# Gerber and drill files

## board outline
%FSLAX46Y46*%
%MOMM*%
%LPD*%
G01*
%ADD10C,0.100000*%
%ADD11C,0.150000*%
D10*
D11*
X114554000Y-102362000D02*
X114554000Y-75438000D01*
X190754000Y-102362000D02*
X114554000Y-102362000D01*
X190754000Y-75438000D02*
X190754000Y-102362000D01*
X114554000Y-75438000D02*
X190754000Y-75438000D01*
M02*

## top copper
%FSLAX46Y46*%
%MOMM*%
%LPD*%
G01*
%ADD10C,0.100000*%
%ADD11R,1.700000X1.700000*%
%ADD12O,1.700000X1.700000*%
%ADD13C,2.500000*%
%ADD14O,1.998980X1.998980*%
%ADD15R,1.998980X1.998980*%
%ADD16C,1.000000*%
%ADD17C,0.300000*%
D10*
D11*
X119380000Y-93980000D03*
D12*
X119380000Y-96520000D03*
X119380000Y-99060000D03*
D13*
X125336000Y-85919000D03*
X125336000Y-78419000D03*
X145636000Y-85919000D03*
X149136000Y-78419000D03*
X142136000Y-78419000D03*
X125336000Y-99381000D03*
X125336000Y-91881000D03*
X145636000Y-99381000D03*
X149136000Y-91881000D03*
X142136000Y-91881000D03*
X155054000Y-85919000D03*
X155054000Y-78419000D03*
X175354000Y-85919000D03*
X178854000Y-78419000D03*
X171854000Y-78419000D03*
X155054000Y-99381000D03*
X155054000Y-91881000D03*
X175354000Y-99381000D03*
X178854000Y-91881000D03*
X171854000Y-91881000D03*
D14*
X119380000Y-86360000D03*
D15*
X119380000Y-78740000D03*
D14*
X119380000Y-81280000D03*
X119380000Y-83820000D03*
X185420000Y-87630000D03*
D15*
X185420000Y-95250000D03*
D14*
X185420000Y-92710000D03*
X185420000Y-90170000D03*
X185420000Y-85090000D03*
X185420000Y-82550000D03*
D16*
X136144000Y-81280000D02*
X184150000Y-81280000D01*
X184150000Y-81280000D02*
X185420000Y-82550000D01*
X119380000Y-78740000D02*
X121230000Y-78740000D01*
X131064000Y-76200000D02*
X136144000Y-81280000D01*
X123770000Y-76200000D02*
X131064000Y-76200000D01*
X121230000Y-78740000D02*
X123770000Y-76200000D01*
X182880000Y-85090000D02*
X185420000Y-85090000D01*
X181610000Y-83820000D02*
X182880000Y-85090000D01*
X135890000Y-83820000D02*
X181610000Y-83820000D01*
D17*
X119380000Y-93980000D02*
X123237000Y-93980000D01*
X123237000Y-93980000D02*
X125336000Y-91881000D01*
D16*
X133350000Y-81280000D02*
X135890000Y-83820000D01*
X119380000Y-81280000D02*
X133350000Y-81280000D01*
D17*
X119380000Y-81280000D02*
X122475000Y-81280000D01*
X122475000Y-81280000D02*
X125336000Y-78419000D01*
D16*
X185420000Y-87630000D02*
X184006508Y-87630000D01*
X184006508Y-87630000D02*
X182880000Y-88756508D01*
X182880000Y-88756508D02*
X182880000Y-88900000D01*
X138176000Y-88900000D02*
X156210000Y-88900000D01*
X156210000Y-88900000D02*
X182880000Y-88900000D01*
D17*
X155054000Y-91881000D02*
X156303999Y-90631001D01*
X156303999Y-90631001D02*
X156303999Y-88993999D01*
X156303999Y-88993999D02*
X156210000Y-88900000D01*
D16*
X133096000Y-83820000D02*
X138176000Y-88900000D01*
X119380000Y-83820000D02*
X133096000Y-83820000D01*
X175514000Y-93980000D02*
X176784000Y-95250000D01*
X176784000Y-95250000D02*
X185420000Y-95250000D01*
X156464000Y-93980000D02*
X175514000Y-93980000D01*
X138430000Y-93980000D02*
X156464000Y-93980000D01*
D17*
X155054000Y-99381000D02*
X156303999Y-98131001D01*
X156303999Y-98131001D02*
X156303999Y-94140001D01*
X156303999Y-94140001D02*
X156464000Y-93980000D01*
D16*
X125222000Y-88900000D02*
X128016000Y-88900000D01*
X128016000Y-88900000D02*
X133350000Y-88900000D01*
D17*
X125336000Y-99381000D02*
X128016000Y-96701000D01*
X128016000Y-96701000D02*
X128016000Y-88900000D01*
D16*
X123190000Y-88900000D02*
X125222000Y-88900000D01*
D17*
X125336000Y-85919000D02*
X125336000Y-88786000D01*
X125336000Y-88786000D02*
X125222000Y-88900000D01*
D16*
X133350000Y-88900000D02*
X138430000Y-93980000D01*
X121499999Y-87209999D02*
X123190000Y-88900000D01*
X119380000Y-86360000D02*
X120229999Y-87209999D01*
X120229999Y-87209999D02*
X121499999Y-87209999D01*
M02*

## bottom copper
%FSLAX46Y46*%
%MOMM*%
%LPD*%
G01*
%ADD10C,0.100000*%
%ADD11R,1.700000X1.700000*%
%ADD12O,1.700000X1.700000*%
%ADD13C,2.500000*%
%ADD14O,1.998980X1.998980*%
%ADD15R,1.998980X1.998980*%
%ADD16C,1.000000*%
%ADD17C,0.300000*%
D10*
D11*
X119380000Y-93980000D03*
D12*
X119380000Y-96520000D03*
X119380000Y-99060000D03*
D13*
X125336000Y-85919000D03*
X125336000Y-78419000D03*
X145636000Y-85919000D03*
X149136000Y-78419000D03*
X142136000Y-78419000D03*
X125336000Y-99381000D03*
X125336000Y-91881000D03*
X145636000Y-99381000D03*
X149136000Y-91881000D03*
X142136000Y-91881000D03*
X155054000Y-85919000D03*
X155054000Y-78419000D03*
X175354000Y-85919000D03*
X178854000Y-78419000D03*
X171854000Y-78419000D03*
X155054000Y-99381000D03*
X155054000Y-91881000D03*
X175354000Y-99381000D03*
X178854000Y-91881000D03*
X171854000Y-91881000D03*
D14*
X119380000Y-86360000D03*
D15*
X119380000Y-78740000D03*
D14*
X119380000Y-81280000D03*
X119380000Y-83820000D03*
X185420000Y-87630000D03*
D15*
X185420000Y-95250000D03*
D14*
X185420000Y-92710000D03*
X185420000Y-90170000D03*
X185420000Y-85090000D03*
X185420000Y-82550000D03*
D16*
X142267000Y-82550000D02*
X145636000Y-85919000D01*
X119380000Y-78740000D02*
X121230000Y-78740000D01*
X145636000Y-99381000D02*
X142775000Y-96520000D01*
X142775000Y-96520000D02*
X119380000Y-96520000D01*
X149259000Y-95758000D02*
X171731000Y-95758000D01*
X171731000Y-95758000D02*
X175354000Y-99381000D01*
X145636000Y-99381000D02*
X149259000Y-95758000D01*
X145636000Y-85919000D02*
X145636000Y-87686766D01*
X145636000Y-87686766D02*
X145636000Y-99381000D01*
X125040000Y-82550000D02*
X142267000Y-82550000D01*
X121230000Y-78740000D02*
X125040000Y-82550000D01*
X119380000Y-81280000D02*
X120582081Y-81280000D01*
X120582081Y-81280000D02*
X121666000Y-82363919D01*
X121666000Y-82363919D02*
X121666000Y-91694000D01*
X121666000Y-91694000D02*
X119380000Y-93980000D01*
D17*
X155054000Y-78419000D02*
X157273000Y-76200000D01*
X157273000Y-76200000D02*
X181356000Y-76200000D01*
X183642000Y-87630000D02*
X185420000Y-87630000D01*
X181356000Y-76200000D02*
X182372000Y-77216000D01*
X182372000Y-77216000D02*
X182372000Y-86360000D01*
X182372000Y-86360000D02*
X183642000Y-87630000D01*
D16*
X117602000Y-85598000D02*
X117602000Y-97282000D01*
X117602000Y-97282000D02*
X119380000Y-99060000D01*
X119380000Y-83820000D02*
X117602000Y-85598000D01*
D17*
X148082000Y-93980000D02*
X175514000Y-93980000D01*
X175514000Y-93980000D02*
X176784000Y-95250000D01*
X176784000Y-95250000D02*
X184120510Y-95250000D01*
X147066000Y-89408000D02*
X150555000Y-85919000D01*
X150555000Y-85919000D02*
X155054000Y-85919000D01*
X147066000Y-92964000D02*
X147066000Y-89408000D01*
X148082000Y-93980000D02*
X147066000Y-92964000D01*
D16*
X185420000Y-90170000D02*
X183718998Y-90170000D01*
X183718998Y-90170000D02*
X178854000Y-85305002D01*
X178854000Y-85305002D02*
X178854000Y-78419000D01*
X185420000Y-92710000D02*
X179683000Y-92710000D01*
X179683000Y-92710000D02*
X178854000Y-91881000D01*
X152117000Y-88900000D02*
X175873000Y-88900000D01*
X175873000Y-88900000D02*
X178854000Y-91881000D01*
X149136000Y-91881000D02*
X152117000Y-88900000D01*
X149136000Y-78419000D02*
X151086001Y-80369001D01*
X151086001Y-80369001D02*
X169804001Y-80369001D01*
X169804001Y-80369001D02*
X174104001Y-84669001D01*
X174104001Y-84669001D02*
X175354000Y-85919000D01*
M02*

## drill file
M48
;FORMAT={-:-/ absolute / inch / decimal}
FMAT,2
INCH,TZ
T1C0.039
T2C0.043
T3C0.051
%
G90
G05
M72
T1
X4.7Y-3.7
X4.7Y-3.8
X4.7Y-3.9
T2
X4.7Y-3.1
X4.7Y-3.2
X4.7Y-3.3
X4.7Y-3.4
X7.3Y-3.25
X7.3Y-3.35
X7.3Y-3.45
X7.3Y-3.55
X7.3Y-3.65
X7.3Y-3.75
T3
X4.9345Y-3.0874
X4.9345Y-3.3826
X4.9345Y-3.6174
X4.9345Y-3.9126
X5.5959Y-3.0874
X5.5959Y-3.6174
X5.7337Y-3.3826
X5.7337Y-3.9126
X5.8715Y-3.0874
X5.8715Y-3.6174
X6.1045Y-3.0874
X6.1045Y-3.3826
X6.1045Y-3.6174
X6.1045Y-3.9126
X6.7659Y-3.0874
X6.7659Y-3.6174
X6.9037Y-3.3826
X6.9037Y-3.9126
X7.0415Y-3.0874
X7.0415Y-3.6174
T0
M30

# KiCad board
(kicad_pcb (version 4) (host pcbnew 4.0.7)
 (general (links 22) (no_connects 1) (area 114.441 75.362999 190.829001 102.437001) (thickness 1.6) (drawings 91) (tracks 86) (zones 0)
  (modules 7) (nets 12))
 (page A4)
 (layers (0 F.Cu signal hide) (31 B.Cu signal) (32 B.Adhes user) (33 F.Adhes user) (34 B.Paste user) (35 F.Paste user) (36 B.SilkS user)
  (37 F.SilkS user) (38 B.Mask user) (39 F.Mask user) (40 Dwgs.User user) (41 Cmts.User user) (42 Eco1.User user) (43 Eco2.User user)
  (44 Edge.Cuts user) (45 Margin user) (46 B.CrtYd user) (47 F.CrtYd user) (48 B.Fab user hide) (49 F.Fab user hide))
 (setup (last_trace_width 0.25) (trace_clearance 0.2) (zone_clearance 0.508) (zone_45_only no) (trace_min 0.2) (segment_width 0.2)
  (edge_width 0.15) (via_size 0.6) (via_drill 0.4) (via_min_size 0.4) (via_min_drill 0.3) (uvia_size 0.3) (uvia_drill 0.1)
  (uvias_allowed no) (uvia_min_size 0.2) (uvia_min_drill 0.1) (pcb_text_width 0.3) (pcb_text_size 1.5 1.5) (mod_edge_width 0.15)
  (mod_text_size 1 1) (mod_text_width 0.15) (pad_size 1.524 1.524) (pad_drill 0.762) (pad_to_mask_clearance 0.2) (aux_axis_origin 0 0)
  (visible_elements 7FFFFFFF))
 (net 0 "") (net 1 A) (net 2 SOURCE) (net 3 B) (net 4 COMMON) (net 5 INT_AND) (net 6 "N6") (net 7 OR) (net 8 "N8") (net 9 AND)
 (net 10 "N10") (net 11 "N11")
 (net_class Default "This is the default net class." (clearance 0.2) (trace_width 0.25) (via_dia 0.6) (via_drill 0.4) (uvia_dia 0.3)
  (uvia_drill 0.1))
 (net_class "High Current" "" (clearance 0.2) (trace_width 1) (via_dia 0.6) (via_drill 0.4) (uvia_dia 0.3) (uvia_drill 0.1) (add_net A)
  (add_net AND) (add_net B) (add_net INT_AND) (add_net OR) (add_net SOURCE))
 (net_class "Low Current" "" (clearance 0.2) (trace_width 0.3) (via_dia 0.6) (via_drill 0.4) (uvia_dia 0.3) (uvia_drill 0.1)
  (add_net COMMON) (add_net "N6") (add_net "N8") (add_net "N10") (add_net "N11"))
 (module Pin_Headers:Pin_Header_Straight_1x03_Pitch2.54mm (layer F.Cu) (at 119.38 93.98)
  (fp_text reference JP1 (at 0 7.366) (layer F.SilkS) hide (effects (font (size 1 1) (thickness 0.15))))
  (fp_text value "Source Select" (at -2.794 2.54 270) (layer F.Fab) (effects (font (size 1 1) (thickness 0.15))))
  (pad 1 thru_hole rect (at 0 0) (size 1.7 1.7) (drill 1) (layers *.Cu *.Mask) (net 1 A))
  (pad 2 thru_hole oval (at 0 2.54) (size 1.7 1.7) (drill 1) (layers *.Cu *.Mask) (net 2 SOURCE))
  (pad 3 thru_hole oval (at 0 5.08) (size 1.7 1.7) (drill 1) (layers *.Cu *.Mask) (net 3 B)))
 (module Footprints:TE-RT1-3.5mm (layer F.Cu) (at 135.636 82.169)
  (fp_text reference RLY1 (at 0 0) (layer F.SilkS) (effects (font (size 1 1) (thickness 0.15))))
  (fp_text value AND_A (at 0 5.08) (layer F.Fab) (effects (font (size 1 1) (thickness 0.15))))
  (pad A2 thru_hole circle (at -10.3 3.75) (size 2.5 2.5) (drill 1.3) (layers *.Cu *.Mask) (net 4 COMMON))
  (pad A1 thru_hole circle (at -10.3 -3.75) (size 2.5 2.5) (drill 1.3) (layers *.Cu *.Mask) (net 1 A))
  (pad 11 thru_hole circle (at 10 3.75) (size 2.5 2.5) (drill 1.3) (layers *.Cu *.Mask) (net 2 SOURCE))
  (pad 14 thru_hole circle (at 13.5 -3.75) (size 2.5 2.5) (drill 1.3) (layers *.Cu *.Mask) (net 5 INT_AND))
  (pad 12 thru_hole circle (at 6.5 -3.75) (size 2.5 2.5) (drill 1.3) (layers *.Cu *.Mask) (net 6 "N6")))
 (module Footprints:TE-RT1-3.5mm (layer F.Cu) (at 135.636 95.631)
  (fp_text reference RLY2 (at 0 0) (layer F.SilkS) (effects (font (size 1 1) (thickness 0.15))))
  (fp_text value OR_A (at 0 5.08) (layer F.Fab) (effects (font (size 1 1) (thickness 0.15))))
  (pad A2 thru_hole circle (at -10.3 3.75) (size 2.5 2.5) (drill 1.3) (layers *.Cu *.Mask) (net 4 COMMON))
  (pad A1 thru_hole circle (at -10.3 -3.75) (size 2.5 2.5) (drill 1.3) (layers *.Cu *.Mask) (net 1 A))
  (pad 11 thru_hole circle (at 10 3.75) (size 2.5 2.5) (drill 1.3) (layers *.Cu *.Mask) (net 2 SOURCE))
  (pad 14 thru_hole circle (at 13.5 -3.75) (size 2.5 2.5) (drill 1.3) (layers *.Cu *.Mask) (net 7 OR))
  (pad 12 thru_hole circle (at 6.5 -3.75) (size 2.5 2.5) (drill 1.3) (layers *.Cu *.Mask) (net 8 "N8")))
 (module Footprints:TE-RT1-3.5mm (layer F.Cu) (at 165.354 82.169)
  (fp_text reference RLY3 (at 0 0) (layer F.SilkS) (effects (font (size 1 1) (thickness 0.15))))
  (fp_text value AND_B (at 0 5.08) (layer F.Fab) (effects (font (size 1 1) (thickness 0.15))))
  (pad A2 thru_hole circle (at -10.3 3.75) (size 2.5 2.5) (drill 1.3) (layers *.Cu *.Mask) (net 4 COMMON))
  (pad A1 thru_hole circle (at -10.3 -3.75) (size 2.5 2.5) (drill 1.3) (layers *.Cu *.Mask) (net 3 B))
  (pad 11 thru_hole circle (at 10 3.75) (size 2.5 2.5) (drill 1.3) (layers *.Cu *.Mask) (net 5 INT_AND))
  (pad 14 thru_hole circle (at 13.5 -3.75) (size 2.5 2.5) (drill 1.3) (layers *.Cu *.Mask) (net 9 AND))
  (pad 12 thru_hole circle (at 6.5 -3.75) (size 2.5 2.5) (drill 1.3) (layers *.Cu *.Mask) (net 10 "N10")))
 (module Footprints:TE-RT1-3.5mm (layer F.Cu) (at 165.354 95.631)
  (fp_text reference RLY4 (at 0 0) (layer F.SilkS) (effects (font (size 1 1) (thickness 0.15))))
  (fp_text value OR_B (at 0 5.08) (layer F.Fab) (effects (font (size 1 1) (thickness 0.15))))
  (pad A2 thru_hole circle (at -10.3 3.75) (size 2.5 2.5) (drill 1.3) (layers *.Cu *.Mask) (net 4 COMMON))
  (pad A1 thru_hole circle (at -10.3 -3.75) (size 2.5 2.5) (drill 1.3) (layers *.Cu *.Mask) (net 3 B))
  (pad 11 thru_hole circle (at 10 3.75) (size 2.5 2.5) (drill 1.3) (layers *.Cu *.Mask) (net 2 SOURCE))
  (pad 14 thru_hole circle (at 13.5 -3.75) (size 2.5 2.5) (drill 1.3) (layers *.Cu *.Mask) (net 7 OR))
  (pad 12 thru_hole circle (at 6.5 -3.75) (size 2.5 2.5) (drill 1.3) (layers *.Cu *.Mask) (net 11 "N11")))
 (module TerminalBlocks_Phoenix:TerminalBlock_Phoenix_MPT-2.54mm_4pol (layer F.Cu) (at 119.38 78.74 270)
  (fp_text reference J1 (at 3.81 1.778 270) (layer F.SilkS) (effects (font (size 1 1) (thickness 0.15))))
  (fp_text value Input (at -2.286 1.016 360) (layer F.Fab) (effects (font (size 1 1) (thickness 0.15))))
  (pad 4 thru_hole oval (at 7.62 0 90) (size 1.99898 1.99898) (drill 1.09728) (layers *.Cu *.Mask) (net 4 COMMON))
  (pad 1 thru_hole rect (at 0 0 90) (size 1.99898 1.99898) (drill 1.09728) (layers *.Cu *.Mask) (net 2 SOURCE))
  (pad 2 thru_hole oval (at 2.54 0 90) (size 1.99898 1.99898) (drill 1.09728) (layers *.Cu *.Mask) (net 1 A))
  (pad 3 thru_hole oval (at 5.08 0 90) (size 1.99898 1.99898) (drill 1.09728) (layers *.Cu *.Mask) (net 3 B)))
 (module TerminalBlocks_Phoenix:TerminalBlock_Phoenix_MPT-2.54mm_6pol (layer F.Cu) (at 185.42 95.25 90)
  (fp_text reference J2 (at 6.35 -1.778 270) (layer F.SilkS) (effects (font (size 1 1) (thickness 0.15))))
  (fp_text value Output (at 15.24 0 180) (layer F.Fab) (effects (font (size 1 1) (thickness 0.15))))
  (pad 4 thru_hole oval (at 7.62 0 270) (size 1.99898 1.99898) (drill 1.09728) (layers *.Cu *.Mask) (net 3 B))
  (pad 1 thru_hole rect (at 0 0 270) (size 1.99898 1.99898) (drill 1.09728) (layers *.Cu *.Mask) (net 4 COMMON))
  (pad 2 thru_hole oval (at 2.54 0 270) (size 1.99898 1.99898) (drill 1.09728) (layers *.Cu *.Mask) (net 7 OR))
  (pad 3 thru_hole oval (at 5.08 0 270) (size 1.99898 1.99898) (drill 1.09728) (layers *.Cu *.Mask) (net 9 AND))
  (pad 5 thru_hole oval (at 10.16 0 270) (size 1.99898 1.99898) (drill 1.09728) (layers *.Cu *.Mask) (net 1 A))
  (pad 6 thru_hole oval (at 12.7 0 270) (size 1.99898 1.99898) (drill 1.09728) (layers *.Cu *.Mask) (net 2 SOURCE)))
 (gr_line (start 114.554 102.362) (end 114.554 75.438) (layer Edge.Cuts) (width 0.15))
 (gr_line (start 190.754 102.362) (end 114.554 102.362) (layer Edge.Cuts) (width 0.15))
 (gr_line (start 190.754 75.438) (end 190.754 102.362) (layer Edge.Cuts) (width 0.15))
 (gr_line (start 114.554 75.438) (end 190.754 75.438) (layer Edge.Cuts) (width 0.15))
 (segment (start 136.144 81.28) (end 184.15 81.28) (width 1) (layer F.Cu) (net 2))
 (segment (start 184.15 81.28) (end 185.42 82.55) (width 1) (layer F.Cu) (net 2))
 (segment (start 119.38 78.74) (end 121.23 78.74) (width 1) (layer F.Cu) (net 2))
 (segment (start 142.267 82.55) (end 145.636 85.919) (width 1) (layer B.Cu) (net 2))
 (segment (start 119.38 78.74) (end 121.23 78.74) (width 1) (layer B.Cu) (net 2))
 (segment (start 145.636 99.381) (end 142.775 96.52) (width 1) (layer B.Cu) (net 2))
 (segment (start 142.775 96.52) (end 119.38 96.52) (width 1) (layer B.Cu) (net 2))
 (segment (start 149.259 95.758) (end 171.731 95.758) (width 1) (layer B.Cu) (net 2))
 (segment (start 171.731 95.758) (end 175.354 99.381) (width 1) (layer B.Cu) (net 2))
 (segment (start 145.636 99.381) (end 149.259 95.758) (width 1) (layer B.Cu) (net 2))
 (segment (start 145.636 85.919) (end 145.636 87.686766) (width 1) (layer B.Cu) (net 2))
 (segment (start 145.636 87.686766) (end 145.636 99.381) (width 1) (layer B.Cu) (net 2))
 (segment (start 131.064 76.2) (end 136.144 81.28) (width 1) (layer F.Cu) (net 2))
 (segment (start 123.77 76.2) (end 131.064 76.2) (width 1) (layer F.Cu) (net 2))
 (segment (start 121.23 78.74) (end 123.77 76.2) (width 1) (layer F.Cu) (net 2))
 (segment (start 125.04 82.55) (end 142.267 82.55) (width 1) (layer B.Cu) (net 2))
 (segment (start 121.23 78.74) (end 125.04 82.55) (width 1) (layer B.Cu) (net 2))
 (segment (start 182.88 85.09) (end 185.42 85.09) (width 1) (layer F.Cu) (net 1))
 (segment (start 181.61 83.82) (end 182.88 85.09) (width 1) (layer F.Cu) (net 1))
 (segment (start 135.89 83.82) (end 181.61 83.82) (width 1) (layer F.Cu) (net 1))
 (segment (start 119.38 93.98) (end 123.237 93.98) (width 0.3) (layer F.Cu) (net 1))
 (segment (start 123.237 93.98) (end 125.336 91.881) (width 0.3) (layer F.Cu) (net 1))
 (segment (start 119.38 81.28) (end 120.582081 81.28) (width 1) (layer B.Cu) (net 1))
 (segment (start 120.582081 81.28) (end 121.666 82.363919) (width 1) (layer B.Cu) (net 1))
 (segment (start 121.666 82.363919) (end 121.666 91.694) (width 1) (layer B.Cu) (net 1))
 (segment (start 121.666 91.694) (end 119.38 93.98) (width 1) (layer B.Cu) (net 1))
 (segment (start 133.35 81.28) (end 135.89 83.82) (width 1) (layer F.Cu) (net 1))
 (segment (start 119.38 81.28) (end 133.35 81.28) (width 1) (layer F.Cu) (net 1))
 (segment (start 119.38 81.28) (end 122.475 81.28) (width 0.3) (layer F.Cu) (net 1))
 (segment (start 122.475 81.28) (end 125.336 78.419) (width 0.3) (layer F.Cu) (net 1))
 (segment (start 185.42 87.63) (end 184.006508 87.63) (width 1) (layer F.Cu) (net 3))
 (segment (start 184.006508 87.63) (end 182.88 88.756508) (width 1) (layer F.Cu) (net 3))
 (segment (start 182.88 88.756508) (end 182.88 88.9) (width 1) (layer F.Cu) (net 3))
 (segment (start 155.054 78.419) (end 157.273 76.2) (width 0.3) (layer B.Cu) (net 3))
 (segment (start 157.273 76.2) (end 181.356 76.2) (width 0.3) (layer B.Cu) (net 3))
 (segment (start 183.642 87.63) (end 185.42 87.63) (width 0.3) (layer B.Cu) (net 3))
 (segment (start 181.356 76.2) (end 182.372 77.216) (width 0.3) (layer B.Cu) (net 3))
 (segment (start 182.372 77.216) (end 182.372 86.36) (width 0.3) (layer B.Cu) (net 3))
 (segment (start 182.372 86.36) (end 183.642 87.63) (width 0.3) (layer B.Cu) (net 3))
 (segment (start 138.176 88.9) (end 156.21 88.9) (width 1) (layer F.Cu) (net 3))
 (segment (start 156.21 88.9) (end 182.88 88.9) (width 1) (layer F.Cu) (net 3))
 (segment (start 155.054 91.881) (end 156.303999 90.631001) (width 0.3) (layer F.Cu) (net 3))
 (segment (start 156.303999 90.631001) (end 156.303999 88.993999) (width 0.3) (layer F.Cu) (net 3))
 (segment (start 156.303999 88.993999) (end 156.21 88.9) (width 0.3) (layer F.Cu) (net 3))
 (segment (start 133.096 83.82) (end 138.176 88.9) (width 1) (layer F.Cu) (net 3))
 (segment (start 119.38 83.82) (end 133.096 83.82) (width 1) (layer F.Cu) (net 3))
 (segment (start 117.602 85.598) (end 117.602 97.282) (width 1) (layer B.Cu) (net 3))
 (segment (start 117.602 97.282) (end 119.38 99.06) (width 1) (layer B.Cu) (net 3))
 (segment (start 119.38 83.82) (end 117.602 85.598) (width 1) (layer B.Cu) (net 3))
 (segment (start 148.082 93.98) (end 175.514 93.98) (width 0.3) (layer B.Cu) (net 4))
 (segment (start 175.514 93.98) (end 176.784 95.25) (width 0.3) (layer B.Cu) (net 4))
 (segment (start 176.784 95.25) (end 184.12051 95.25) (width 0.3) (layer B.Cu) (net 4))
 (segment (start 175.514 93.98) (end 176.784 95.25) (width 1) (layer F.Cu) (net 4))
 (segment (start 176.784 95.25) (end 185.42 95.25) (width 1) (layer F.Cu) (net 4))
 (segment (start 156.464 93.98) (end 175.514 93.98) (width 1) (layer F.Cu) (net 4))
 (segment (start 147.066 89.408) (end 150.555 85.919) (width 0.3) (layer B.Cu) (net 4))
 (segment (start 150.555 85.919) (end 155.054 85.919) (width 0.3) (layer B.Cu) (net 4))
 (segment (start 147.066 92.964) (end 147.066 89.408) (width 0.3) (layer B.Cu) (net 4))
 (segment (start 148.082 93.98) (end 147.066 92.964) (width 0.3) (layer B.Cu) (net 4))
 (segment (start 138.43 93.98) (end 156.464 93.98) (width 1) (layer F.Cu) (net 4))
 (segment (start 155.054 99.381) (end 156.303999 98.131001) (width 0.3) (layer F.Cu) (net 4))
 (segment (start 156.303999 98.131001) (end 156.303999 94.140001) (width 0.3) (layer F.Cu) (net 4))
 (segment (start 156.303999 94.140001) (end 156.464 93.98) (width 0.3) (layer F.Cu) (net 4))
 (segment (start 125.222 88.9) (end 128.016 88.9) (width 1) (layer F.Cu) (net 4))
 (segment (start 128.016 88.9) (end 133.35 88.9) (width 1) (layer F.Cu) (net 4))
 (segment (start 125.336 99.381) (end 128.016 96.701) (width 0.3) (layer F.Cu) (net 4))
 (segment (start 128.016 96.701) (end 128.016 88.9) (width 0.3) (layer F.Cu) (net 4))
 (segment (start 123.19 88.9) (end 125.222 88.9) (width 1) (layer F.Cu) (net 4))
 (segment (start 125.336 85.919) (end 125.336 88.786) (width 0.3) (layer F.Cu) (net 4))
 (segment (start 125.336 88.786) (end 125.222 88.9) (width 0.3) (layer F.Cu) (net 4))
 (segment (start 133.35 88.9) (end 138.43 93.98) (width 1) (layer F.Cu) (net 4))
 (segment (start 121.499999 87.209999) (end 123.19 88.9) (width 1) (layer F.Cu) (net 4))
 (segment (start 119.38 86.36) (end 120.229999 87.209999) (width 1) (layer F.Cu) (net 4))
 (segment (start 120.229999 87.209999) (end 121.499999 87.209999) (width 1) (layer F.Cu) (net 4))
 (segment (start 185.42 90.17) (end 183.718998 90.17) (width 1) (layer B.Cu) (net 9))
 (segment (start 183.718998 90.17) (end 178.854 85.305002) (width 1) (layer B.Cu) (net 9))
 (segment (start 178.854 85.305002) (end 178.854 78.419) (width 1) (layer B.Cu) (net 9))
 (segment (start 185.42 92.71) (end 179.683 92.71) (width 1) (layer B.Cu) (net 7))
 (segment (start 179.683 92.71) (end 178.854 91.881) (width 1) (layer B.Cu) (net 7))
 (segment (start 152.117 88.9) (end 175.873 88.9) (width 1) (layer B.Cu) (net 7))
 (segment (start 175.873 88.9) (end 178.854 91.881) (width 1) (layer B.Cu) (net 7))
 (segment (start 149.136 91.881) (end 152.117 88.9) (width 1) (layer B.Cu) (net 7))
 (segment (start 149.136 78.419) (end 151.086001 80.369001) (width 1) (layer B.Cu) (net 5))
 (segment (start 151.086001 80.369001) (end 169.804001 80.369001) (width 1) (layer B.Cu) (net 5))
 (segment (start 169.804001 80.369001) (end 174.104001 84.669001) (width 1) (layer B.Cu) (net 5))
 (segment (start 174.104001 84.669001) (end 175.354 85.919) (width 1) (layer B.Cu) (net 5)))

